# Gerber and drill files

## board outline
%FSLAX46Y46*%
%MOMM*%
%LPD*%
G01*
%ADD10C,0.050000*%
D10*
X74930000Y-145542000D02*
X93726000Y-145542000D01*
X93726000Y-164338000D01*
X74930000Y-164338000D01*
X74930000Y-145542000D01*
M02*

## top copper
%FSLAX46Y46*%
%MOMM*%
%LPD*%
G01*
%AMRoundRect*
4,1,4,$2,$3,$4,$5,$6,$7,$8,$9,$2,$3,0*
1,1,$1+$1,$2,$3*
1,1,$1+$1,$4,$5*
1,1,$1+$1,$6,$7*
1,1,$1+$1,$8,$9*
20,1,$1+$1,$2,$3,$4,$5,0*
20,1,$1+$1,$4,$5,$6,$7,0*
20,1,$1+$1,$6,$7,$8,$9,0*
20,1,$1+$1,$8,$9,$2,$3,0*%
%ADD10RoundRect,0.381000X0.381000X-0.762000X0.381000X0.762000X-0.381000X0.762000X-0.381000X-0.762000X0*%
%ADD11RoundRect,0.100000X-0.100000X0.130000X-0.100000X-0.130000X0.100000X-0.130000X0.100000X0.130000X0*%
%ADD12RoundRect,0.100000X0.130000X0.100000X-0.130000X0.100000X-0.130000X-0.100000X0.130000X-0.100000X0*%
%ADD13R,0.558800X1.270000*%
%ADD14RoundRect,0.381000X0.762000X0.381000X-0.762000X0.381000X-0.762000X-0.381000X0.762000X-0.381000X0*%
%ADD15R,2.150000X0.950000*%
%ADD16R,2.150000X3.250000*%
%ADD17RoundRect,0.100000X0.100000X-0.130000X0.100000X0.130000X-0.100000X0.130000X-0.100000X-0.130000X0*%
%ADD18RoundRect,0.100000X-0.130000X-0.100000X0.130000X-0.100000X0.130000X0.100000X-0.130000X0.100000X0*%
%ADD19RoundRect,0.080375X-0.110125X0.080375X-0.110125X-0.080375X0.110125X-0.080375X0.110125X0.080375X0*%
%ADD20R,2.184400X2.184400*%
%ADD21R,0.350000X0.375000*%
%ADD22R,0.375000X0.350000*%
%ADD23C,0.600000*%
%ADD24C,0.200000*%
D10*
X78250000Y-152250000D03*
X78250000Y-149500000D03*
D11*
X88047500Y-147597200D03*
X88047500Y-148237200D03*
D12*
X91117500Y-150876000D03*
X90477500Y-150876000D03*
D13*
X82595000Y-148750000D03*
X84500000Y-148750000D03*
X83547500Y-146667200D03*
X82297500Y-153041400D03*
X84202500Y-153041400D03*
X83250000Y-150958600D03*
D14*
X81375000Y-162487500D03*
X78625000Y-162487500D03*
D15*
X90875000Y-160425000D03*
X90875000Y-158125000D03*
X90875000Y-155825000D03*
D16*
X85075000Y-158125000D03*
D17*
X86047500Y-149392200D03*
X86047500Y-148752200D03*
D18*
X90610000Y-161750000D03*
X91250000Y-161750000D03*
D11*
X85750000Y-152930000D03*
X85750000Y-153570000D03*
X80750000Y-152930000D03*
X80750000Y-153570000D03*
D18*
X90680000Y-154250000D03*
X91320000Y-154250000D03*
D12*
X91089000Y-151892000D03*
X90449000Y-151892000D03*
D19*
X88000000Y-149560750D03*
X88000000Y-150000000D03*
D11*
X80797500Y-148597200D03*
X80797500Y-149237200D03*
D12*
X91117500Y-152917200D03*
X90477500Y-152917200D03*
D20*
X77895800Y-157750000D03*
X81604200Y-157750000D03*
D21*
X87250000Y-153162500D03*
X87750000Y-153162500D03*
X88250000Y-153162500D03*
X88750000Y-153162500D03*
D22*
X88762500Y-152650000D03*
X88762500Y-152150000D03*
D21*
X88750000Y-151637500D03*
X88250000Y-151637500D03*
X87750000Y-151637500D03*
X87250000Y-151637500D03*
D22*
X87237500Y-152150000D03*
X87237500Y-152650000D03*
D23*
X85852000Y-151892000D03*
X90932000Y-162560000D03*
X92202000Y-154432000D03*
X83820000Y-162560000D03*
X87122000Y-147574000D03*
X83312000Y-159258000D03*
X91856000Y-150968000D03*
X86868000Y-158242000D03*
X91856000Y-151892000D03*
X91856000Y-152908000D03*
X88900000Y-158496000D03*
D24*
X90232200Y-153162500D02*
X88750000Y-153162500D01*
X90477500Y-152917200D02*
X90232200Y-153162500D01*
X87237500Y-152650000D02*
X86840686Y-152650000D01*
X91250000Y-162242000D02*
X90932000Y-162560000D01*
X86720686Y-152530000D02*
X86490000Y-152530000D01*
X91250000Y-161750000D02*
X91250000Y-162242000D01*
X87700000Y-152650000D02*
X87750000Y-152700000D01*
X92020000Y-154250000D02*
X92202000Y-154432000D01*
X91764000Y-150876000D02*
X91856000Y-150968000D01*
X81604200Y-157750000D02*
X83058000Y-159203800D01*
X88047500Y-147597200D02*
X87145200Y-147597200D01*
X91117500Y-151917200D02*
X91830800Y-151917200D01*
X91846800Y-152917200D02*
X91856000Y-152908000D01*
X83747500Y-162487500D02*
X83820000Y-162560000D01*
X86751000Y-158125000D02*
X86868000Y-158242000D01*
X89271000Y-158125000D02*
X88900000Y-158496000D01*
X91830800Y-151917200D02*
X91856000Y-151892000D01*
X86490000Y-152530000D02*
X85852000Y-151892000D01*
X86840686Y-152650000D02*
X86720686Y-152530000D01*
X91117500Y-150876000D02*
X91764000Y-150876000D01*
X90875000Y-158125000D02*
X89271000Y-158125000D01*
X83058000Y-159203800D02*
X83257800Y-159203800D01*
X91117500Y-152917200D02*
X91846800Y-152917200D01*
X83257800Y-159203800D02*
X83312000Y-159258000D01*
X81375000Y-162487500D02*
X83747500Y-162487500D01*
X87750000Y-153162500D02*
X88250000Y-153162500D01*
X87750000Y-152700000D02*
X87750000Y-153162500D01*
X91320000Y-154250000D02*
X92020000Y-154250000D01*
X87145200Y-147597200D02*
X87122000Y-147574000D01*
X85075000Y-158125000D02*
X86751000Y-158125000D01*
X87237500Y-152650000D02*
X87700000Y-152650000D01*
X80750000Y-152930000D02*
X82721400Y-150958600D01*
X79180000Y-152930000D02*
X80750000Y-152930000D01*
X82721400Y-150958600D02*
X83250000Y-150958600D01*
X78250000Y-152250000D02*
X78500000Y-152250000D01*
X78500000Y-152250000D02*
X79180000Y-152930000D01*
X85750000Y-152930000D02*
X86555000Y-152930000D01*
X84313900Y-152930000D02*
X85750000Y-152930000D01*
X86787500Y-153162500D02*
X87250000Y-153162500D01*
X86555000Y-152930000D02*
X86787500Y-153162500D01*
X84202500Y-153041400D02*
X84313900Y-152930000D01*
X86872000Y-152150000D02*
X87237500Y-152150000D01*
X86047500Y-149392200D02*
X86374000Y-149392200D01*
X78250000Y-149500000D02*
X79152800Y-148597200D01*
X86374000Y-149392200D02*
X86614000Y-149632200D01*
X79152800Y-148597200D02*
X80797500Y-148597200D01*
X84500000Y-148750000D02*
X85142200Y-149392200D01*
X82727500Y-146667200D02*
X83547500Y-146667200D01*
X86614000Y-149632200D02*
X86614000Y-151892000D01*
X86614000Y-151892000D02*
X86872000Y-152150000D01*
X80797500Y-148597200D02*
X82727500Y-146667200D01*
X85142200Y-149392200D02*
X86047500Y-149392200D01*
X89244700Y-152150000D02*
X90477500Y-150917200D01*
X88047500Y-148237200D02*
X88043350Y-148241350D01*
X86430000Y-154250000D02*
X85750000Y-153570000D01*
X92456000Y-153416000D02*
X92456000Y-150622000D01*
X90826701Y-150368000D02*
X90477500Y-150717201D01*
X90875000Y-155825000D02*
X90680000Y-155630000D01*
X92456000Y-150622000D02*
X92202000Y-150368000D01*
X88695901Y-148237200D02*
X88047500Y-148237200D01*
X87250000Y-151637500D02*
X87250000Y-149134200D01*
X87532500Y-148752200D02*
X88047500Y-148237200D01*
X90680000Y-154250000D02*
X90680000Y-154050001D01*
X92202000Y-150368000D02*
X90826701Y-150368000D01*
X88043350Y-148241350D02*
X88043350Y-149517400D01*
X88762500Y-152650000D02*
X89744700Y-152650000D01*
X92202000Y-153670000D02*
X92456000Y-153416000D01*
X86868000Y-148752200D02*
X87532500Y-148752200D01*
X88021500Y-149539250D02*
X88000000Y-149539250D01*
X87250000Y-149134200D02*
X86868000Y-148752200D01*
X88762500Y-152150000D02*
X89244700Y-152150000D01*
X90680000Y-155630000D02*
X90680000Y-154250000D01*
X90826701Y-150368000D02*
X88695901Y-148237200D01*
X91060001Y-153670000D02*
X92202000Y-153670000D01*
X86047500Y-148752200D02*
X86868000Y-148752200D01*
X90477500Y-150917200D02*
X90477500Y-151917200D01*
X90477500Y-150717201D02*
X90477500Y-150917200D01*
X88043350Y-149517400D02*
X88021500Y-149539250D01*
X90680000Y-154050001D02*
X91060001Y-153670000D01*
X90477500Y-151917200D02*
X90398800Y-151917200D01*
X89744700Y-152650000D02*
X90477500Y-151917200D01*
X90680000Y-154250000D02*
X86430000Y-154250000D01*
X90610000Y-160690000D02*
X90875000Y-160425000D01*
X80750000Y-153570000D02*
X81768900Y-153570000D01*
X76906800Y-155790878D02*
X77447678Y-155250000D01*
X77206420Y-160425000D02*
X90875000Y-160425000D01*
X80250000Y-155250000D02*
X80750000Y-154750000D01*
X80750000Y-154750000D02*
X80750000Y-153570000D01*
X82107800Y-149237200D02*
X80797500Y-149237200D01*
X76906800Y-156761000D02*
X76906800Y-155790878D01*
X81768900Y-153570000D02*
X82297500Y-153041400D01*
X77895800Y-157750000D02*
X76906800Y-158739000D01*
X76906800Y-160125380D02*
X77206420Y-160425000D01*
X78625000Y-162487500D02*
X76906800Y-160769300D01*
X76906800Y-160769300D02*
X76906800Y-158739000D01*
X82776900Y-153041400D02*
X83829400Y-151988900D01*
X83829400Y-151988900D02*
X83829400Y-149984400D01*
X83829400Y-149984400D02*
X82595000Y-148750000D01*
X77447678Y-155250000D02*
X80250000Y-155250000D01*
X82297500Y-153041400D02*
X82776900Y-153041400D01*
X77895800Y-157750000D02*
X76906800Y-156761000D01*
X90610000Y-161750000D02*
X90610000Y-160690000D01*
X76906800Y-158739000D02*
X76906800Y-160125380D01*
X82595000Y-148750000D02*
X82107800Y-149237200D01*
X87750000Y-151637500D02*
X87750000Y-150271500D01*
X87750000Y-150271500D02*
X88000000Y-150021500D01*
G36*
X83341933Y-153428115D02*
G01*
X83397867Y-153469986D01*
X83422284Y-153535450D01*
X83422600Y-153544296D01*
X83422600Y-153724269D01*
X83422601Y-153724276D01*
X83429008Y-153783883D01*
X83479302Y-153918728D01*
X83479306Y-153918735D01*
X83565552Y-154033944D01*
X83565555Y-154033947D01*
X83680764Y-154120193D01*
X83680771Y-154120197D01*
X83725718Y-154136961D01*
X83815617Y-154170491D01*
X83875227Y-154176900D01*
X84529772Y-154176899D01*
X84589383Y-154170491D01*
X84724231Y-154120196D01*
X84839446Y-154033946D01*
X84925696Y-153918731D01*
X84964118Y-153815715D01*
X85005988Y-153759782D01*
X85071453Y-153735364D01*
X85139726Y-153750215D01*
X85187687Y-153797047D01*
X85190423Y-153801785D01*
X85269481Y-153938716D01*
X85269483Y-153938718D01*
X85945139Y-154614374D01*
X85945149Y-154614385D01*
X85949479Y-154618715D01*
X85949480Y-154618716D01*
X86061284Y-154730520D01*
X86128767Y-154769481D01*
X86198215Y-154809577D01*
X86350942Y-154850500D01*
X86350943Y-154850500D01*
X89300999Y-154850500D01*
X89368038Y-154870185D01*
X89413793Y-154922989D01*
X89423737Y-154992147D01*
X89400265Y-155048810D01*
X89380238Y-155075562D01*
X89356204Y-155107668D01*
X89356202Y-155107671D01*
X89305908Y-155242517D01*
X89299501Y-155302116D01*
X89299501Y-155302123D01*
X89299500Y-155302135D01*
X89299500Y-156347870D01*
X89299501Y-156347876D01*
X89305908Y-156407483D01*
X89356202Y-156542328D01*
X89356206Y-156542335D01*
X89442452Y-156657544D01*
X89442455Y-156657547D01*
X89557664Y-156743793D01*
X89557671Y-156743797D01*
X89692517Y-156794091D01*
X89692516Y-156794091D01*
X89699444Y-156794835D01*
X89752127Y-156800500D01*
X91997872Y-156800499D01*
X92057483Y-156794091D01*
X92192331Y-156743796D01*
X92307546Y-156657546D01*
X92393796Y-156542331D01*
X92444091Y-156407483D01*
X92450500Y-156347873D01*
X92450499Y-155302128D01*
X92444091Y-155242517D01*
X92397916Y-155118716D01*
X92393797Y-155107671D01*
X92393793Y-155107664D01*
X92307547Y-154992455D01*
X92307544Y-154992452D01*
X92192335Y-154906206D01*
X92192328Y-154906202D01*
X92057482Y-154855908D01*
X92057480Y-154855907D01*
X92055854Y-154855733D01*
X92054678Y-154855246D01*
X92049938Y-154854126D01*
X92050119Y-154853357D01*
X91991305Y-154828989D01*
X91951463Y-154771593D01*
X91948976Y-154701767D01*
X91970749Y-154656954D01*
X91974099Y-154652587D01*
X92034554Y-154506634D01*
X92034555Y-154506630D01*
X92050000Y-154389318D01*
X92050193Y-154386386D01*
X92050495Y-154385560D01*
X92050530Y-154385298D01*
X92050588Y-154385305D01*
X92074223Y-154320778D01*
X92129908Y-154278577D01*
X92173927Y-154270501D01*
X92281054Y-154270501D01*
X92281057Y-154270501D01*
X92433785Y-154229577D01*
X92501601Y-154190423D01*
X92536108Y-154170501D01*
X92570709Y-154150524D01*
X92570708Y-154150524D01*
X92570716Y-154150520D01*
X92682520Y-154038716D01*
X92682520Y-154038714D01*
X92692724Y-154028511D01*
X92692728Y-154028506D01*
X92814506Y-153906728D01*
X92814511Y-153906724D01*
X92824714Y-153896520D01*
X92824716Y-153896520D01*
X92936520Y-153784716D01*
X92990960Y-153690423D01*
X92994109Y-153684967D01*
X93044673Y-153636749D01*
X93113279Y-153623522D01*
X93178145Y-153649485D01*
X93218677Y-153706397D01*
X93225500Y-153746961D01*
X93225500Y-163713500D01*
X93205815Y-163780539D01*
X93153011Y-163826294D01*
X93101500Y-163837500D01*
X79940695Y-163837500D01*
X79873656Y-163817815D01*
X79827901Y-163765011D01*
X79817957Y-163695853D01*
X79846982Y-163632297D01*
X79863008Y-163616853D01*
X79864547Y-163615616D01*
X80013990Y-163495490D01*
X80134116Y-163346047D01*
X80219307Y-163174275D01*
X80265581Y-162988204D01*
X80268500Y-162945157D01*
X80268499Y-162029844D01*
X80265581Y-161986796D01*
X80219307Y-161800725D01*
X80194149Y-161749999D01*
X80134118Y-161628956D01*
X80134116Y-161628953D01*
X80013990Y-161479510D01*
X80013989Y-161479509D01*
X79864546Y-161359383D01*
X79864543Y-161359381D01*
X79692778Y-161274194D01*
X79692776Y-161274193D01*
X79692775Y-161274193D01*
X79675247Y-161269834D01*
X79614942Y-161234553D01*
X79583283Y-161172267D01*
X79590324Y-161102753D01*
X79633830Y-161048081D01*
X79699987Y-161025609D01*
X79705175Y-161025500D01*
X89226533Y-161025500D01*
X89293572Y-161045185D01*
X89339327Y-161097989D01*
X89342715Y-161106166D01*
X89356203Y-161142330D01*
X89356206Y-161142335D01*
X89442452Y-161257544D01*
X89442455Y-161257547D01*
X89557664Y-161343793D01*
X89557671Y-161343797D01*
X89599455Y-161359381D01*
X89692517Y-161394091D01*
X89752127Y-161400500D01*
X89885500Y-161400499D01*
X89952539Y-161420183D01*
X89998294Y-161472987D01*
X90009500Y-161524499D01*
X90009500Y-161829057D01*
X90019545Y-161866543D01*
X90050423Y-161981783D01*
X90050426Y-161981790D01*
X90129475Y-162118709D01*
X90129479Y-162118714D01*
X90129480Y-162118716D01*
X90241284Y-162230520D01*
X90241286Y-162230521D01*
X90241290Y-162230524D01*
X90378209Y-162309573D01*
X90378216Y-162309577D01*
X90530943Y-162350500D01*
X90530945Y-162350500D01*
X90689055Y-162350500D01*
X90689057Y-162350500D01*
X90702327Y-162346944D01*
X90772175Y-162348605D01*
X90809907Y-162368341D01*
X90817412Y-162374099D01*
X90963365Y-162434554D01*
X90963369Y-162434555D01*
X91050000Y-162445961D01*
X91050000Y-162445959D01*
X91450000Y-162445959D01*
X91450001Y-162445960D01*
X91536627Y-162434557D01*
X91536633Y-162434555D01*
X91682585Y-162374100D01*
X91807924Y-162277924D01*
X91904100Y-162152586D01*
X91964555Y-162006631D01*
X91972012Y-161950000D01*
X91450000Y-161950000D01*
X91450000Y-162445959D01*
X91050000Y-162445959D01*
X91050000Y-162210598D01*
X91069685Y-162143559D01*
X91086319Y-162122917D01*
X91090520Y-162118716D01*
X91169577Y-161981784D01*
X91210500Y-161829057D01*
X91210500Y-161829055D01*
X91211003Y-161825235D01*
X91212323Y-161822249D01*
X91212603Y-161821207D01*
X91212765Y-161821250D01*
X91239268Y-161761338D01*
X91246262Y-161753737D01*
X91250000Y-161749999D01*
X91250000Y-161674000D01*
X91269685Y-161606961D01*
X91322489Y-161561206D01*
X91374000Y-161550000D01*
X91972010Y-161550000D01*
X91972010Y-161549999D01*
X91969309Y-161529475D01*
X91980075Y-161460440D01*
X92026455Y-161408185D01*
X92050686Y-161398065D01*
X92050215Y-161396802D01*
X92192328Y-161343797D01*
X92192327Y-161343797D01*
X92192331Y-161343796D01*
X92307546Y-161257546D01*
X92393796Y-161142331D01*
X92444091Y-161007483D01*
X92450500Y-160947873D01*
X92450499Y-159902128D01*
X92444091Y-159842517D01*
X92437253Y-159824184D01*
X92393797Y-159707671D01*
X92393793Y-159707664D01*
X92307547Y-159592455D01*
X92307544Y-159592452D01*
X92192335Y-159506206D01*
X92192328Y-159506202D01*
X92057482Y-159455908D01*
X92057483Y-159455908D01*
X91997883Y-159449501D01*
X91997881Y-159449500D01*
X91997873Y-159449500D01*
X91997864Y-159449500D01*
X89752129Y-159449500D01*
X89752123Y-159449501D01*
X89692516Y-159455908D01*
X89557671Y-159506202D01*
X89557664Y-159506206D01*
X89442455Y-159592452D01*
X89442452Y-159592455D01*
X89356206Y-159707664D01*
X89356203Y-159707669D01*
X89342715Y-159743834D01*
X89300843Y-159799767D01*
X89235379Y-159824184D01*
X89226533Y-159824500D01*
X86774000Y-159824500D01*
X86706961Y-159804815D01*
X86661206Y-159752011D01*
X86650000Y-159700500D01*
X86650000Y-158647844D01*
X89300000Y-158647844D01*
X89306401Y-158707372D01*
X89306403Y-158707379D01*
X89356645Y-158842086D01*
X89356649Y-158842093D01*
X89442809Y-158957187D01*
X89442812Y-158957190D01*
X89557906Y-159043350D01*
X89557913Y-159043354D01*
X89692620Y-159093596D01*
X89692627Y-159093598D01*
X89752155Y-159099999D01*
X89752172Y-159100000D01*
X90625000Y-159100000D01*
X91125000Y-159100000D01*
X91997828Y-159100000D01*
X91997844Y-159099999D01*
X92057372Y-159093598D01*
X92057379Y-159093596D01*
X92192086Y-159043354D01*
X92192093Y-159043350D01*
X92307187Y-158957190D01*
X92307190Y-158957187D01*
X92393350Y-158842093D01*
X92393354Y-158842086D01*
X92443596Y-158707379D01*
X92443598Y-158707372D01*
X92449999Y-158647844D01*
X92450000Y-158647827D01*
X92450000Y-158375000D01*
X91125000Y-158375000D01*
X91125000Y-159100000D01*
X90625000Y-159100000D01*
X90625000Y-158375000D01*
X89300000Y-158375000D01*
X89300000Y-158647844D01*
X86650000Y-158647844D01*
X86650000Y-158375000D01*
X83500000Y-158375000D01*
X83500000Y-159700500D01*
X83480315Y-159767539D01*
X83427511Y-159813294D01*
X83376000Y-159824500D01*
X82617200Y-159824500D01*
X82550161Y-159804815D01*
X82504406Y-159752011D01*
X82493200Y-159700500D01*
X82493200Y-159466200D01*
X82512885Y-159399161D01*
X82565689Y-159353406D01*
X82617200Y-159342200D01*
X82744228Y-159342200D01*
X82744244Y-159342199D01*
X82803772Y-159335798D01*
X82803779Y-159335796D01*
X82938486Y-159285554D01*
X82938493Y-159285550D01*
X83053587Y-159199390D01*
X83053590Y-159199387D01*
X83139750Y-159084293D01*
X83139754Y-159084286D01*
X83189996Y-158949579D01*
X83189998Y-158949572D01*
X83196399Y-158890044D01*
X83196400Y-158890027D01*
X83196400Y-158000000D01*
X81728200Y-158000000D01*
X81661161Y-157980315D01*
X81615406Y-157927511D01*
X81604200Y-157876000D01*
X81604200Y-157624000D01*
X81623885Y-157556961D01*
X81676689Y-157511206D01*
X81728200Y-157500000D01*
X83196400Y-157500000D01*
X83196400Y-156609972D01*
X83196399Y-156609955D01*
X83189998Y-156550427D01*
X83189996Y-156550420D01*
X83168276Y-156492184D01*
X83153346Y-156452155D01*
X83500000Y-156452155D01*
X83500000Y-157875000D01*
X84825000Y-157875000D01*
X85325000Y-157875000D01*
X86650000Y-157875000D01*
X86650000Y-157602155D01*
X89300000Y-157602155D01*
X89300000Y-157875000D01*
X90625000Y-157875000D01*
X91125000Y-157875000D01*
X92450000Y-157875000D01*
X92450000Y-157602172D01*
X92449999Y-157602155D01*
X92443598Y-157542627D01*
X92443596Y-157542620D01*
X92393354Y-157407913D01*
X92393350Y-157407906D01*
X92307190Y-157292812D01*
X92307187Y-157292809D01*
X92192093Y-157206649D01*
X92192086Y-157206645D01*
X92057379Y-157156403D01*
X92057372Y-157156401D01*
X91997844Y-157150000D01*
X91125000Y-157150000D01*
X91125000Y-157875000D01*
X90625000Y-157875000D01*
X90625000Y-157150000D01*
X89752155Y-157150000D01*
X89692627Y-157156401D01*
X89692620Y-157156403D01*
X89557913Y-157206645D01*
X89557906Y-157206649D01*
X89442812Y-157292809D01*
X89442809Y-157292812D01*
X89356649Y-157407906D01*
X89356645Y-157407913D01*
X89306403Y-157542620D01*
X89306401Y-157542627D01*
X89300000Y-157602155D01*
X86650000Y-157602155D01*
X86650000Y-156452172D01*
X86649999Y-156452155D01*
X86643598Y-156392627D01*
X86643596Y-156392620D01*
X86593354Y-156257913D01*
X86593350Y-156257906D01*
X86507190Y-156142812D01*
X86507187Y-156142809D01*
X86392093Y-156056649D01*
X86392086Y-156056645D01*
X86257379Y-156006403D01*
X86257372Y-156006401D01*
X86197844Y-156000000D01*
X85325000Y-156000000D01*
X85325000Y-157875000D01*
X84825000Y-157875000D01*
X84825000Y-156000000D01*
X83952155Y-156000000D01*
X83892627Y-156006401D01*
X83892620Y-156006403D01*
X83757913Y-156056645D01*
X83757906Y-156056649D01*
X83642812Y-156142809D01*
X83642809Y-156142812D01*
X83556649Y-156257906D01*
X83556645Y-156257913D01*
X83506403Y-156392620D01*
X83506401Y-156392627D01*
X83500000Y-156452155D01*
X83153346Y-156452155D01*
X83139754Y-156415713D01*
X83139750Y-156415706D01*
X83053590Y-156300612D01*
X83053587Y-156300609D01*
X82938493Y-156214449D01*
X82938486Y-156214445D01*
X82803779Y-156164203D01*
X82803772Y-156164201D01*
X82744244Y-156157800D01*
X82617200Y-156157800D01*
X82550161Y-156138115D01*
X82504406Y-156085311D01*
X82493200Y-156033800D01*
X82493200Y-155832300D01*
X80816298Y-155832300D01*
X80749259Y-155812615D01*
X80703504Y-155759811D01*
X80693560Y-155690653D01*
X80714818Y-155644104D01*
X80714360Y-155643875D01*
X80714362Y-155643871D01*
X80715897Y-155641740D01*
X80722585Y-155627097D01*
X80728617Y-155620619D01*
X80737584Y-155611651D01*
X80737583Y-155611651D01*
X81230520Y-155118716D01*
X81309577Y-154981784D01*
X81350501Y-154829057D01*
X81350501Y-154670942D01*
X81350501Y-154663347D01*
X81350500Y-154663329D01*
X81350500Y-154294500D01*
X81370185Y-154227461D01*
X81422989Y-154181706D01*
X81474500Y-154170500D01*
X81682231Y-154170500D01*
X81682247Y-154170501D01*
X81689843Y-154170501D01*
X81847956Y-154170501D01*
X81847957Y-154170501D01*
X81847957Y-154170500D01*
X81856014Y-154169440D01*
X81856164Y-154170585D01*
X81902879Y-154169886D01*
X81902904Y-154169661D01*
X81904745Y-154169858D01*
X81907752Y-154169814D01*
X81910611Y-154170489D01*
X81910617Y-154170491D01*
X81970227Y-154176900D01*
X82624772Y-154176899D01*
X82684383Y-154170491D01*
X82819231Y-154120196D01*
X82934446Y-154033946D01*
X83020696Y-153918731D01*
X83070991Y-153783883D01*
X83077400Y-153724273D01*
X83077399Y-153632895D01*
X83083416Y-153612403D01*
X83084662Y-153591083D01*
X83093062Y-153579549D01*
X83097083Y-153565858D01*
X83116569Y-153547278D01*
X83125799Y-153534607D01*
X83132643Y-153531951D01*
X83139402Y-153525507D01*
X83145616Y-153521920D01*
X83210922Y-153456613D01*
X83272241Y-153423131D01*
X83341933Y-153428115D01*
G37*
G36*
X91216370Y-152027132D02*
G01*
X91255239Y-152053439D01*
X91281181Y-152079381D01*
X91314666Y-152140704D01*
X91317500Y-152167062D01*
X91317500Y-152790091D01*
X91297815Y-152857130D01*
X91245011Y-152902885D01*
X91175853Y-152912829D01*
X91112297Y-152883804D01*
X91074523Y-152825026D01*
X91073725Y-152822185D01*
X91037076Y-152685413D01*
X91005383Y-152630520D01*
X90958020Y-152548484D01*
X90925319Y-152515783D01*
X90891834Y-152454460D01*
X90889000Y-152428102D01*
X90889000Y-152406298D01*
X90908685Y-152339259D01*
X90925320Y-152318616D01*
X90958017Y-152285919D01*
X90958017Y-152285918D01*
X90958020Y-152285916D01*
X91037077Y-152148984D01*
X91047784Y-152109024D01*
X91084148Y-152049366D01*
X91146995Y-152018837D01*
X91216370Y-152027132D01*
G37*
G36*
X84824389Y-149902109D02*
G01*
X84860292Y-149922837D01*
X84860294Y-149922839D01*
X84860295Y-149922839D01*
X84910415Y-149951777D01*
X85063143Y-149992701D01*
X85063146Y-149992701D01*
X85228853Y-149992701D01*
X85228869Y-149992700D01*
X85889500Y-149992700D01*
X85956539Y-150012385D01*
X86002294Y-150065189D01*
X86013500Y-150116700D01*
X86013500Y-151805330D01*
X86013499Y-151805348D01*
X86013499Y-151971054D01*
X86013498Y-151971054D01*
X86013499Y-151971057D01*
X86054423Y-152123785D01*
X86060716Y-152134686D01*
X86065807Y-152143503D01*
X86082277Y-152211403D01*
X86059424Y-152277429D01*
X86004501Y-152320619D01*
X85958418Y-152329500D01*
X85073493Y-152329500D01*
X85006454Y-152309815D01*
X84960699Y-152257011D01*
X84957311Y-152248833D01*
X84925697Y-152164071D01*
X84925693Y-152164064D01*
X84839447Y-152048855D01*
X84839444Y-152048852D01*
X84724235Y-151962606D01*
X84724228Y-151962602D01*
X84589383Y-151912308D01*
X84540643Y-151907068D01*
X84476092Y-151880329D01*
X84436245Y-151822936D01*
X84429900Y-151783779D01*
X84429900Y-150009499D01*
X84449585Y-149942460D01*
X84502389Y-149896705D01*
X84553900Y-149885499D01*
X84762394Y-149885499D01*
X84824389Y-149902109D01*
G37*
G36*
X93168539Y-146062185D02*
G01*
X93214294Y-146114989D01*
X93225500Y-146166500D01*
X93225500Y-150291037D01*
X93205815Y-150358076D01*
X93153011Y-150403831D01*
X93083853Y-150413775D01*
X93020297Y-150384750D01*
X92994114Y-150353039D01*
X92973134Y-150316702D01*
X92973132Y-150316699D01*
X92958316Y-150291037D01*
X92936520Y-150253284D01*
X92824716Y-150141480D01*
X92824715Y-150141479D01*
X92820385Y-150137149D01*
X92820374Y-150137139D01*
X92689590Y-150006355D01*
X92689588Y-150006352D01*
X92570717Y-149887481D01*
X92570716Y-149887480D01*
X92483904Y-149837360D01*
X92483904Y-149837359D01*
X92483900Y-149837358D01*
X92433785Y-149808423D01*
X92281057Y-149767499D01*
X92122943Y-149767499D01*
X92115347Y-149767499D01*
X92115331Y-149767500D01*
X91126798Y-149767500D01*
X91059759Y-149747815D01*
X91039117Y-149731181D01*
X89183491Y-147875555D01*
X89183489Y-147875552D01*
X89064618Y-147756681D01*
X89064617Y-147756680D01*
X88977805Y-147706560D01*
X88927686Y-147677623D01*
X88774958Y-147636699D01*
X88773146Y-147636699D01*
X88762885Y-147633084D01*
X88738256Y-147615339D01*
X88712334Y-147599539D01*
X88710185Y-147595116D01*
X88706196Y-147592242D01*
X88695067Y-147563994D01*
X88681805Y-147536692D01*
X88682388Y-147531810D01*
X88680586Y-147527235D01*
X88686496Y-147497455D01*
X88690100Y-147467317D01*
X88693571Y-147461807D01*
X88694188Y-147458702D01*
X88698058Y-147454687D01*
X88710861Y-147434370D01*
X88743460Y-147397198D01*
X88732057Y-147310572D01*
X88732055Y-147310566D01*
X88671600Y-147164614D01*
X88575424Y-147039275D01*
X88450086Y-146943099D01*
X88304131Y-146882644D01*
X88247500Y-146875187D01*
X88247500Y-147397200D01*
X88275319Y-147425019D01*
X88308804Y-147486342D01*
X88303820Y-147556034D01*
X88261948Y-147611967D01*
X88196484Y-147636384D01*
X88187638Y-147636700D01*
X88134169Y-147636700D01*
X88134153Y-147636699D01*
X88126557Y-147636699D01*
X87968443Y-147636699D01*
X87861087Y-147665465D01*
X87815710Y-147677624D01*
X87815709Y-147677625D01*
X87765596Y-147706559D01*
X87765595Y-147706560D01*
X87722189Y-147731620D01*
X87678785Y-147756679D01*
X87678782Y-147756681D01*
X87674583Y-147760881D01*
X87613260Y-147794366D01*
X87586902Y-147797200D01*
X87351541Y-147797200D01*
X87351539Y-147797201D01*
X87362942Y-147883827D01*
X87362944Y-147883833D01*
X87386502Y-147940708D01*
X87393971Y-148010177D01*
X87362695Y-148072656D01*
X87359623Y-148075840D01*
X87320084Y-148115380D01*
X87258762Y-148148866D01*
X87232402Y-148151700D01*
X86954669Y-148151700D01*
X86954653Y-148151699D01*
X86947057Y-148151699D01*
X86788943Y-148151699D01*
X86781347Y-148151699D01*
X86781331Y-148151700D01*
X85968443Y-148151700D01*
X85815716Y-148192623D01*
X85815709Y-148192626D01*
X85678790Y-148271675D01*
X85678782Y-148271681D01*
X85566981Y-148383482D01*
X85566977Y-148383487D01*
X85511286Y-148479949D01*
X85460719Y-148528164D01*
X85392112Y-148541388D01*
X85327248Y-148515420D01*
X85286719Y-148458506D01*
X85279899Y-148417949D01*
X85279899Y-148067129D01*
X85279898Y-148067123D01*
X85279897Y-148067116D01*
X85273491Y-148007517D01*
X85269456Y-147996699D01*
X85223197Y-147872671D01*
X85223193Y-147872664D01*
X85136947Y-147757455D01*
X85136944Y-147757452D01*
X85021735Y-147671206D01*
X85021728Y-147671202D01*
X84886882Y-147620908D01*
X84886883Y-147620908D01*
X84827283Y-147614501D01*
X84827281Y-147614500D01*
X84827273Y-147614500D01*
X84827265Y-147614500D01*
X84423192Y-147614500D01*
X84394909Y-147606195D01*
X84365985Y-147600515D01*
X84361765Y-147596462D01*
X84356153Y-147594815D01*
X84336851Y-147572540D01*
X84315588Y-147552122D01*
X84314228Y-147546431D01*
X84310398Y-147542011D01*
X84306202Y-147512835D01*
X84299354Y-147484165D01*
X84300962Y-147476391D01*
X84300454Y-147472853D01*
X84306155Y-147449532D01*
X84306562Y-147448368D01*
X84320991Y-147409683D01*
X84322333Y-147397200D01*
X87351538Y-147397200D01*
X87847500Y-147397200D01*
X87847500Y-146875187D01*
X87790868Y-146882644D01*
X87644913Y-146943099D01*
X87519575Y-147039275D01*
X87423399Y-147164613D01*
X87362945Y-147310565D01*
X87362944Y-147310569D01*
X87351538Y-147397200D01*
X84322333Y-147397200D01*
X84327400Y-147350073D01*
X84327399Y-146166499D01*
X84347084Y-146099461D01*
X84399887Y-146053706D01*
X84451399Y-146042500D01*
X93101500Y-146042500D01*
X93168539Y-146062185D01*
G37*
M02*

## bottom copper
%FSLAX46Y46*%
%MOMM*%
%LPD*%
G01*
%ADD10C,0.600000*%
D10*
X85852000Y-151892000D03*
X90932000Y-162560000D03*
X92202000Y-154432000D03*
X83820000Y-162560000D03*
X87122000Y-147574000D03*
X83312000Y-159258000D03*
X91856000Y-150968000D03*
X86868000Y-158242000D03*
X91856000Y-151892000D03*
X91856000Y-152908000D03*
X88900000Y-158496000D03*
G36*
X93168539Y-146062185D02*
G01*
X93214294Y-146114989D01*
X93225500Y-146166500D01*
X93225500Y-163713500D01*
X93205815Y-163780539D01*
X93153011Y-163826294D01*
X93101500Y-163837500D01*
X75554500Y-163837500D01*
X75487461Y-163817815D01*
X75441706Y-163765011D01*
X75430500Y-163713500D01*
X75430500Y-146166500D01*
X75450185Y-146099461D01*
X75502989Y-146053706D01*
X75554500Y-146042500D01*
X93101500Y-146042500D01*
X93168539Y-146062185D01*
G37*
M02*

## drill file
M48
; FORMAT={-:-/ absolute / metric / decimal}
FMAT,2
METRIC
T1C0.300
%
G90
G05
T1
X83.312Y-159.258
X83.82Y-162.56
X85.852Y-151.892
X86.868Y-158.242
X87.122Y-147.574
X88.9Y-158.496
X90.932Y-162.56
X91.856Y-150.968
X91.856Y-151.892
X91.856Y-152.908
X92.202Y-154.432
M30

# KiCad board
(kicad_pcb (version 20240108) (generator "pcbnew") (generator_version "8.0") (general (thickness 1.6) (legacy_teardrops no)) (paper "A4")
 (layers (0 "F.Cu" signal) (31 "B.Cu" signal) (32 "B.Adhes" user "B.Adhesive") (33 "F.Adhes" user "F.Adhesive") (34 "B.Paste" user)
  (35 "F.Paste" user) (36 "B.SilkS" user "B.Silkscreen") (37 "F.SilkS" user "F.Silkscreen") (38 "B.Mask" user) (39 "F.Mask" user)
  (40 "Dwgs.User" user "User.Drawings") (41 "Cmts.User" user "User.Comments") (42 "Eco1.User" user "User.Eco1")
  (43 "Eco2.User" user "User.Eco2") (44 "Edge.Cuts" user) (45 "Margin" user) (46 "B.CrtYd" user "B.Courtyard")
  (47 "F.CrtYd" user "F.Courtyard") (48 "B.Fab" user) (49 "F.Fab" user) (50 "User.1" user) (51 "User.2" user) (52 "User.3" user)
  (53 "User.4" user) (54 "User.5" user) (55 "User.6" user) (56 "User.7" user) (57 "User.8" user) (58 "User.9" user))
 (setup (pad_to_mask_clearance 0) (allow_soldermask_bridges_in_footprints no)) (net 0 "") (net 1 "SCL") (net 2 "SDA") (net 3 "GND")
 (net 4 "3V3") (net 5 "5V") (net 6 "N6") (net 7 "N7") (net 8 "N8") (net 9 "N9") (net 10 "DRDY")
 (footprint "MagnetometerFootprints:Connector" (layer "F.Cu") (at 81.5 149.25 90)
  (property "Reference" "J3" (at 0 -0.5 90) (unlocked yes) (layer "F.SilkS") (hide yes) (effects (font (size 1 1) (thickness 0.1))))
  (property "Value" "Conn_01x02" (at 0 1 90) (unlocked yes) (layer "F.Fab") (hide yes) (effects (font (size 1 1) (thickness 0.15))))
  (pad "1" smd roundrect (at -3 -3.25 90) (size 2.286 1.524) (layers "F.Cu" "F.Mask") (roundrect_rratio 0.25) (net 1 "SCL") (zone_connect 2)
   (thermal_bridge_angle 45))
  (pad "2" smd roundrect (at -0.25 -3.25 90) (size 2.286 1.524) (layers "F.Cu" "F.Mask") (roundrect_rratio 0.25) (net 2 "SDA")
   (zone_connect 2) (thermal_bridge_angle 45)))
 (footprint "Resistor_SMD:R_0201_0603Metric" (layer "F.Cu") (at 88.0475 147.9172 -90)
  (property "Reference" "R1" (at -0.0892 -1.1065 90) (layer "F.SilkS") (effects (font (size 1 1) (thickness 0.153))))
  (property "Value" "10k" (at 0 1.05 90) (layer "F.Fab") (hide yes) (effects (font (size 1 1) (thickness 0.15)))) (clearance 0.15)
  (pad "" smd roundrect (at -0.345 0 270) (size 0.318 0.36) (layers "F.Paste") (roundrect_rratio 0.25))
  (pad "" smd roundrect (at 0.345 0 270) (size 0.318 0.36) (layers "F.Paste") (roundrect_rratio 0.25))
  (pad "1" smd roundrect (at -0.32 0 270) (size 0.46 0.4) (layers "F.Cu" "F.Mask") (roundrect_rratio 0.25) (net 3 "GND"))
  (pad "2" smd roundrect (at 0.32 0 270) (size 0.46 0.4) (layers "F.Cu" "F.Mask") (roundrect_rratio 0.25) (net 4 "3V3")))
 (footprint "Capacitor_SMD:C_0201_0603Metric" (layer "F.Cu") (at 90.7975 150.876 180)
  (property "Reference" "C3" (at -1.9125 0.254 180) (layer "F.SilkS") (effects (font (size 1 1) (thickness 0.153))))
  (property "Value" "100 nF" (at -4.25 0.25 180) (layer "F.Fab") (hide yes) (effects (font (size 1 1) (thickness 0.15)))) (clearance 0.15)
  (pad "" smd roundrect (at -0.345 0 180) (size 0.318 0.36) (layers "F.Paste") (roundrect_rratio 0.25))
  (pad "" smd roundrect (at 0.345 0 180) (size 0.318 0.36) (layers "F.Paste") (roundrect_rratio 0.25))
  (pad "1" smd roundrect (at -0.32 0 180) (size 0.46 0.4) (layers "F.Cu" "F.Mask") (roundrect_rratio 0.25) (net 3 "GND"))
  (pad "2" smd roundrect (at 0.32 0 180) (size 0.46 0.4) (layers "F.Cu" "F.Mask") (roundrect_rratio 0.25) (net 4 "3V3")))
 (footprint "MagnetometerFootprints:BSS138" (layer "F.Cu") (at 83.5475 147.7086)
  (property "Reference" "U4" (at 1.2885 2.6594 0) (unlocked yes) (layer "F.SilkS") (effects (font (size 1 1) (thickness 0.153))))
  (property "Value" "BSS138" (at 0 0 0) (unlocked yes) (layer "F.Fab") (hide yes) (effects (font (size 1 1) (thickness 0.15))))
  (pad "1" smd rect (at -0.9525 1.0414) (size 0.5588 1.27) (layers "F.Cu" "F.Paste" "F.Mask") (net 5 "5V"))
  (pad "2" smd rect (at 0.9525 1.0414) (size 0.5588 1.27) (layers "F.Cu" "F.Paste" "F.Mask") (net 2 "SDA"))
  (pad "3" smd rect (at 0 -1.0414) (size 0.5588 1.27) (layers "F.Cu" "F.Paste" "F.Mask") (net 2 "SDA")))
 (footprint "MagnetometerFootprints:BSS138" (layer "F.Cu") (at 83.25 152)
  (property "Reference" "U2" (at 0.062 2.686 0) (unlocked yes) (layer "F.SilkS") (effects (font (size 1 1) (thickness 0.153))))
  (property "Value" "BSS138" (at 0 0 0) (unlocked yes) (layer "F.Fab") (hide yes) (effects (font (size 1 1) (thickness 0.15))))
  (pad "1" smd rect (at -0.9525 1.0414) (size 0.5588 1.27) (layers "F.Cu" "F.Paste" "F.Mask") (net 5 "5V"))
  (pad "2" smd rect (at 0.9525 1.0414) (size 0.5588 1.27) (layers "F.Cu" "F.Paste" "F.Mask") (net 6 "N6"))
  (pad "3" smd rect (at 0 -1.0414) (size 0.5588 1.27) (layers "F.Cu" "F.Paste" "F.Mask") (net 1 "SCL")))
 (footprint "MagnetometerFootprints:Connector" (layer "F.Cu") (at 78.375 159.2375 180)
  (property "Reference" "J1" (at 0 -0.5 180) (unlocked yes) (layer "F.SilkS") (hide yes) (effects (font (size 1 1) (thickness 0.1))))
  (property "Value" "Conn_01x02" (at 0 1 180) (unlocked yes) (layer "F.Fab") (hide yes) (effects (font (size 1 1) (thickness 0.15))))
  (pad "1" smd roundrect (at -3 -3.25 180) (size 2.286 1.524) (layers "F.Cu" "F.Mask") (roundrect_rratio 0.25) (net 3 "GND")
   (zone_connect 2) (thermal_bridge_angle 45))
  (pad "2" smd roundrect (at -0.25 -3.25 180) (size 2.286 1.524) (layers "F.Cu" "F.Mask") (roundrect_rratio 0.25) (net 5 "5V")
   (zone_connect 2) (thermal_bridge_angle 45)))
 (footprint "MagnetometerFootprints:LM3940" (layer "F.Cu") (at 87.5 155 180)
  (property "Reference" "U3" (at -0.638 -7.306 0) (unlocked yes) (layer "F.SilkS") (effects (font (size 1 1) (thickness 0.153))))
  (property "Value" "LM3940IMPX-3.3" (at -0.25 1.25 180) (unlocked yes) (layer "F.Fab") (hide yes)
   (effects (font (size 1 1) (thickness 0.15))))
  (pad "1" smd rect (at -3.375 -5.425 180) (size 2.15 0.95) (layers "F.Cu" "F.Paste" "F.Mask") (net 5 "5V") (solder_mask_margin 0.102))
  (pad "2" smd rect (at -3.375 -3.125 180) (size 2.15 0.95) (layers "F.Cu" "F.Paste" "F.Mask") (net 3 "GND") (solder_mask_margin 0.102))
  (pad "3" smd rect (at -3.375 -0.825 180) (size 2.15 0.95) (layers "F.Cu" "F.Paste" "F.Mask") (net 4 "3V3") (solder_mask_margin 0.102))
  (pad "4" smd rect (at 2.425 -3.125 180) (size 2.15 3.25) (layers "F.Cu" "F.Paste" "F.Mask") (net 3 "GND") (solder_mask_margin 0.102)))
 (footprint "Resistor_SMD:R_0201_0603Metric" (layer "F.Cu") (at 86.0475 149.0722 90)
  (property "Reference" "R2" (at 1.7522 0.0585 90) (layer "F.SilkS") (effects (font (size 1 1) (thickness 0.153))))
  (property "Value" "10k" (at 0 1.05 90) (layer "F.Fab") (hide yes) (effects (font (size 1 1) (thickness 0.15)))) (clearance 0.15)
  (pad "" smd roundrect (at -0.345 0 90) (size 0.318 0.36) (layers "F.Paste") (roundrect_rratio 0.25))
  (pad "" smd roundrect (at 0.345 0 90) (size 0.318 0.36) (layers "F.Paste") (roundrect_rratio 0.25))
  (pad "1" smd roundrect (at -0.32 0 90) (size 0.46 0.4) (layers "F.Cu" "F.Mask") (roundrect_rratio 0.25) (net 2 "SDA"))
  (pad "2" smd roundrect (at 0.32 0 90) (size 0.46 0.4) (layers "F.Cu" "F.Mask") (roundrect_rratio 0.25) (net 4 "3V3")))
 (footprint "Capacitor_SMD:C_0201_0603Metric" (layer "F.Cu") (at 90.93 161.75)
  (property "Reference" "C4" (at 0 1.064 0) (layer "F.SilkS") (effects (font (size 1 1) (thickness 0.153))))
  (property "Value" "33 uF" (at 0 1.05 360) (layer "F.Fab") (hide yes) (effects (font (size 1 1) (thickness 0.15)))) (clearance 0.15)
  (pad "" smd roundrect (at -0.345 0) (size 0.318 0.36) (layers "F.Paste") (roundrect_rratio 0.25))
  (pad "" smd roundrect (at 0.345 0) (size 0.318 0.36) (layers "F.Paste") (roundrect_rratio 0.25))
  (pad "1" smd roundrect (at -0.32 0) (size 0.46 0.4) (layers "F.Cu" "F.Mask") (roundrect_rratio 0.25) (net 5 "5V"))
  (pad "2" smd roundrect (at 0.32 0) (size 0.46 0.4) (layers "F.Cu" "F.Mask") (roundrect_rratio 0.25) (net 3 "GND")))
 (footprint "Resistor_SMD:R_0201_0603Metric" (layer "F.Cu") (at 85.75 153.25 -90)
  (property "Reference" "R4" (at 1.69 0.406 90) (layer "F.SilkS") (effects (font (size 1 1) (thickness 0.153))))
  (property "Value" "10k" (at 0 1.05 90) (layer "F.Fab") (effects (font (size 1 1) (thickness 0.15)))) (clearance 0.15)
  (pad "" smd roundrect (at -0.345 0 270) (size 0.318 0.36) (layers "F.Paste") (roundrect_rratio 0.25))
  (pad "" smd roundrect (at 0.345 0 270) (size 0.318 0.36) (layers "F.Paste") (roundrect_rratio 0.25))
  (pad "1" smd roundrect (at -0.32 0 270) (size 0.46 0.4) (layers "F.Cu" "F.Mask") (roundrect_rratio 0.25) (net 6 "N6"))
  (pad "2" smd roundrect (at 0.32 0 270) (size 0.46 0.4) (layers "F.Cu" "F.Mask") (roundrect_rratio 0.25) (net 4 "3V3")))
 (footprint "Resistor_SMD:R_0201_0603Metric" (layer "F.Cu") (at 80.75 153.25 -90)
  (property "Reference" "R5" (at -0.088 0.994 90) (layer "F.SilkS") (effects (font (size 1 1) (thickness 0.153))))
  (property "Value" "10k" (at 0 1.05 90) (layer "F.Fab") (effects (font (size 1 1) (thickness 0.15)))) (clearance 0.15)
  (pad "" smd roundrect (at -0.345 0 270) (size 0.318 0.36) (layers "F.Paste") (roundrect_rratio 0.25))
  (pad "" smd roundrect (at 0.345 0 270) (size 0.318 0.36) (layers "F.Paste") (roundrect_rratio 0.25))
  (pad "1" smd roundrect (at -0.32 0 270) (size 0.46 0.4) (layers "F.Cu" "F.Mask") (roundrect_rratio 0.25) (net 1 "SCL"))
  (pad "2" smd roundrect (at 0.32 0 270) (size 0.46 0.4) (layers "F.Cu" "F.Mask") (roundrect_rratio 0.25) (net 5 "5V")))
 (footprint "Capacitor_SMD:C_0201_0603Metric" (layer "F.Cu") (at 91 154.25)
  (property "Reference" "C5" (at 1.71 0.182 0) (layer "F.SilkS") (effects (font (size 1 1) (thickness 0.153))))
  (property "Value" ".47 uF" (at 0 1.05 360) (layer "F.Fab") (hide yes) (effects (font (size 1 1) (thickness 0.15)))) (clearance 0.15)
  (pad "" smd roundrect (at -0.345 0) (size 0.318 0.36) (layers "F.Paste") (roundrect_rratio 0.25))
  (pad "" smd roundrect (at 0.345 0) (size 0.318 0.36) (layers "F.Paste") (roundrect_rratio 0.25))
  (pad "1" smd roundrect (at -0.32 0) (size 0.46 0.4) (layers "F.Cu" "F.Mask") (roundrect_rratio 0.25) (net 4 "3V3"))
  (pad "2" smd roundrect (at 0.32 0) (size 0.46 0.4) (layers "F.Cu" "F.Mask") (roundrect_rratio 0.25) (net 3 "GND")))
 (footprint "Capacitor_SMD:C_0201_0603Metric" (layer "F.Cu") (at 90.769 151.892 180)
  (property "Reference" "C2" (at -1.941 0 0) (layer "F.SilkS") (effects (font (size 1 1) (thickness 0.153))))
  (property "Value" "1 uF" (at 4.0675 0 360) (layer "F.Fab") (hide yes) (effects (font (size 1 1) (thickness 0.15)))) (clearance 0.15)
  (pad "" smd roundrect (at -0.345 0 180) (size 0.318 0.36) (layers "F.Paste") (roundrect_rratio 0.25))
  (pad "" smd roundrect (at 0.345 0 180) (size 0.318 0.36) (layers "F.Paste") (roundrect_rratio 0.25))
  (pad "1" smd roundrect (at -0.32 0 180) (size 0.46 0.4) (layers "F.Cu" "F.Mask") (roundrect_rratio 0.25) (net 3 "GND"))
  (pad "2" smd roundrect (at 0.32 0 180) (size 0.46 0.4) (layers "F.Cu" "F.Mask") (roundrect_rratio 0.25) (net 4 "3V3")))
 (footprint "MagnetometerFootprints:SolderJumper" (layer "F.Cu") (at 85.8095 153.9 -90)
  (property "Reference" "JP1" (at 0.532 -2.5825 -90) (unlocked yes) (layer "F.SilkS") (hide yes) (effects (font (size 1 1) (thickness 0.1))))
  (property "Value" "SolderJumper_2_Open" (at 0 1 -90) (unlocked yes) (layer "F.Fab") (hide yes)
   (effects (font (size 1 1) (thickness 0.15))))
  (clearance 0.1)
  (pad "1" smd roundrect (at -4.33925 -2.1905 270) (size 0.3215 0.381) (layers "F.Cu" "F.Paste" "F.Mask") (roundrect_rratio 0.25)
   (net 4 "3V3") (thermal_bridge_angle 45))
  (pad "2" smd roundrect (at -3.9 -2.1905 270) (size 0.3215 0.381) (layers "F.Cu" "F.Paste" "F.Mask") (roundrect_rratio 0.25) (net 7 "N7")
   (thermal_bridge_angle 45)))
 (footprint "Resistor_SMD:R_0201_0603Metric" (layer "F.Cu") (at 80.7975 148.9172 -90)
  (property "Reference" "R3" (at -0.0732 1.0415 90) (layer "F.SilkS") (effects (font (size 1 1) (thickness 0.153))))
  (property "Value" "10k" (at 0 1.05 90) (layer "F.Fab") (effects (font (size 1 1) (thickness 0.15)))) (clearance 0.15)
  (pad "" smd roundrect (at -0.345 0 270) (size 0.318 0.36) (layers "F.Paste") (roundrect_rratio 0.25))
  (pad "" smd roundrect (at 0.345 0 270) (size 0.318 0.36) (layers "F.Paste") (roundrect_rratio 0.25))
  (pad "1" smd roundrect (at -0.32 0 270) (size 0.46 0.4) (layers "F.Cu" "F.Mask") (roundrect_rratio 0.25) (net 2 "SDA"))
  (pad "2" smd roundrect (at 0.32 0 270) (size 0.46 0.4) (layers "F.Cu" "F.Mask") (roundrect_rratio 0.25) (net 5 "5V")))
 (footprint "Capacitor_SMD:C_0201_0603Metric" (layer "F.Cu") (at 90.7975 152.9172 180)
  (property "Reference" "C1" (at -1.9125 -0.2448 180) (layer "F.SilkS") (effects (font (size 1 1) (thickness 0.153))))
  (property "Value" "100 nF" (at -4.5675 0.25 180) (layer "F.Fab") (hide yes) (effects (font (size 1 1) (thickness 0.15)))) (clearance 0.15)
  (pad "" smd roundrect (at -0.345 0 180) (size 0.318 0.36) (layers "F.Paste") (roundrect_rratio 0.25))
  (pad "" smd roundrect (at 0.345 0 180) (size 0.318 0.36) (layers "F.Paste") (roundrect_rratio 0.25))
  (pad "1" smd roundrect (at -0.32 0 180) (size 0.46 0.4) (layers "F.Cu" "F.Mask") (roundrect_rratio 0.25) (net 3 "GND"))
  (pad "2" smd roundrect (at 0.32 0 180) (size 0.46 0.4) (layers "F.Cu" "F.Mask") (roundrect_rratio 0.25) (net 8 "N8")))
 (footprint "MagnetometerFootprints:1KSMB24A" (layer "F.Cu") (at 79.75 157.75)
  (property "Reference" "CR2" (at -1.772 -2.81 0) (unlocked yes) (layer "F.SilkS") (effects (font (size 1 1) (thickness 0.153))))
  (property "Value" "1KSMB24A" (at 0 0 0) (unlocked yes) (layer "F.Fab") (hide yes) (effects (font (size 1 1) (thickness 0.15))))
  (pad "1" smd rect (at -1.8542 0 90) (size 2.1844 2.1844) (layers "F.Cu" "F.Paste" "F.Mask") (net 5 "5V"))
  (pad "2" smd rect (at 1.8542 0 90) (size 2.1844 2.1844) (layers "F.Cu" "F.Paste" "F.Mask") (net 3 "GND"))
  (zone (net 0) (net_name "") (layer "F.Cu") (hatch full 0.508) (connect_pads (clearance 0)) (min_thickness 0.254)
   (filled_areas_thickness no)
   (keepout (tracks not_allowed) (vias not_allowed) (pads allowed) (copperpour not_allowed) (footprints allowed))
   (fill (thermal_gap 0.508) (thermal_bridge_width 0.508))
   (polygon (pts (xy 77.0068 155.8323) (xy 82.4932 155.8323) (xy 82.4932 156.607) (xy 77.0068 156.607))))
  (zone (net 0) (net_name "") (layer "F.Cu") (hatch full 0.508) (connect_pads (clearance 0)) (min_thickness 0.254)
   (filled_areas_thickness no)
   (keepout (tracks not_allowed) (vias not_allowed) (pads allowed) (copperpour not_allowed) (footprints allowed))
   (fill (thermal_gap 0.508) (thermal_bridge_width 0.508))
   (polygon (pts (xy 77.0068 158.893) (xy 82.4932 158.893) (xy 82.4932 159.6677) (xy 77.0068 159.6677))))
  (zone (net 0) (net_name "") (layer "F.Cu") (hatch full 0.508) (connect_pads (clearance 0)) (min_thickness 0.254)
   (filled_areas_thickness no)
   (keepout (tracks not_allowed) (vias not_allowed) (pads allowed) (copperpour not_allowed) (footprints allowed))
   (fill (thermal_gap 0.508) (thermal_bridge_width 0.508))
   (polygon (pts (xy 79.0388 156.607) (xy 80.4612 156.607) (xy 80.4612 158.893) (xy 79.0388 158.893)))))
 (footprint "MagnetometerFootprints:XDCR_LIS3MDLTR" (layer "F.Cu") (at 88 152.4 90)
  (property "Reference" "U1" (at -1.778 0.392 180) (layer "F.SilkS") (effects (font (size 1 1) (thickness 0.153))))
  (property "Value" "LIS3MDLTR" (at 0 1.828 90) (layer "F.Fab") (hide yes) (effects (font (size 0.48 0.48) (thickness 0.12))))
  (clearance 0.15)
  (pad "1" smd rect (at -0.7625 -0.75 90) (size 0.375 0.35) (layers "F.Cu" "F.Paste") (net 6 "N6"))
  (pad "2" smd rect (at -0.7625 -0.25 90) (size 0.375 0.35) (layers "F.Cu" "F.Paste") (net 3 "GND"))
  (pad "3" smd rect (at -0.7625 0.25 90) (size 0.375 0.35) (layers "F.Cu" "F.Paste") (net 3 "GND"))
  (pad "4" smd rect (at -0.7625 0.75 90) (size 0.375 0.35) (layers "F.Cu" "F.Paste") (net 8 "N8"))
  (pad "5" smd rect (at -0.25 0.7625 90) (size 0.35 0.375) (layers "F.Cu" "F.Paste") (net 4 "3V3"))
  (pad "6" smd rect (at 0.25 0.7625 90) (size 0.35 0.375) (layers "F.Cu" "F.Paste") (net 4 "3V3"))
  (pad "7" smd rect (at 0.7625 0.75 90) (size 0.375 0.35) (layers "F.Cu" "F.Paste") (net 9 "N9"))
  (pad "8" smd rect (at 0.7625 0.25 90) (size 0.375 0.35) (layers "F.Cu" "F.Paste") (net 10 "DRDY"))
  (pad "9" smd rect (at 0.7625 -0.25 90) (size 0.375 0.35) (layers "F.Cu" "F.Paste") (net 7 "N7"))
  (pad "10" smd rect (at 0.7625 -0.75 90) (size 0.375 0.35) (layers "F.Cu" "F.Paste") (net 4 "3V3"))
  (pad "11" smd rect (at 0.25 -0.7625 90) (size 0.35 0.375) (layers "F.Cu" "F.Paste") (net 2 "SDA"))
  (pad "12" smd rect (at -0.25 -0.7625 90) (size 0.35 0.375) (layers "F.Cu" "F.Paste") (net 3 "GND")))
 (gr_rect (start 74.93 145.542) (end 93.726 164.338) (stroke (width 0.05) (type default)) (fill none) (layer "Edge.Cuts"))
 (segment (start 90.2322 153.1625) (end 88.75 153.1625) (width 0.2) (layer "F.Cu") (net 8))
 (segment (start 90.4775 152.9172) (end 90.2322 153.1625) (width 0.2) (layer "F.Cu") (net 8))
 (segment (start 87.2375 152.65) (end 86.840686 152.65) (width 0.2) (layer "F.Cu") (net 3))
 (segment (start 91.25 162.242) (end 90.932 162.56) (width 0.2) (layer "F.Cu") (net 3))
 (segment (start 86.720686 152.53) (end 86.49 152.53) (width 0.2) (layer "F.Cu") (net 3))
 (segment (start 91.25 161.75) (end 91.25 162.242) (width 0.2) (layer "F.Cu") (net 3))
 (segment (start 87.7 152.65) (end 87.75 152.7) (width 0.2) (layer "F.Cu") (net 3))
 (segment (start 92.02 154.25) (end 92.202 154.432) (width 0.2) (layer "F.Cu") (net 3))
 (segment (start 91.764 150.876) (end 91.856 150.968) (width 0.2) (layer "F.Cu") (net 3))
 (segment (start 81.6042 157.75) (end 83.058 159.2038) (width 0.2) (layer "F.Cu") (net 3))
 (segment (start 88.0475 147.5972) (end 87.1452 147.5972) (width 0.2) (layer "F.Cu") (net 3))
 (segment (start 91.1175 151.9172) (end 91.8308 151.9172) (width 0.2) (layer "F.Cu") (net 3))
 (segment (start 91.8468 152.9172) (end 91.856 152.908) (width 0.2) (layer "F.Cu") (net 3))
 (segment (start 83.7475 162.4875) (end 83.82 162.56) (width 0.2) (layer "F.Cu") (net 3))
 (segment (start 86.751 158.125) (end 86.868 158.242) (width 0.2) (layer "F.Cu") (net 3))
 (segment (start 89.271 158.125) (end 88.9 158.496) (width 0.2) (layer "F.Cu") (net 3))
 (segment (start 91.8308 151.9172) (end 91.856 151.892) (width 0.2) (layer "F.Cu") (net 3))
 (segment (start 86.49 152.53) (end 85.852 151.892) (width 0.2) (layer "F.Cu") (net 3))
 (segment (start 86.840686 152.65) (end 86.720686 152.53) (width 0.2) (layer "F.Cu") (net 3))
 (segment (start 91.1175 150.876) (end 91.764 150.876) (width 0.2) (layer "F.Cu") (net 3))
 (segment (start 90.875 158.125) (end 89.271 158.125) (width 0.2) (layer "F.Cu") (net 3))
 (segment (start 83.058 159.2038) (end 83.2578 159.2038) (width 0.2) (layer "F.Cu") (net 3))
 (segment (start 91.1175 152.9172) (end 91.8468 152.9172) (width 0.2) (layer "F.Cu") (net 3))
 (segment (start 83.2578 159.2038) (end 83.312 159.258) (width 0.2) (layer "F.Cu") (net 3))
 (segment (start 81.375 162.4875) (end 83.7475 162.4875) (width 0.2) (layer "F.Cu") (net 3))
 (segment (start 87.75 153.1625) (end 88.25 153.1625) (width 0.2) (layer "F.Cu") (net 3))
 (segment (start 87.75 152.7) (end 87.75 153.1625) (width 0.2) (layer "F.Cu") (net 3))
 (segment (start 91.32 154.25) (end 92.02 154.25) (width 0.2) (layer "F.Cu") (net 3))
 (segment (start 87.1452 147.5972) (end 87.122 147.574) (width 0.2) (layer "F.Cu") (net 3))
 (segment (start 85.075 158.125) (end 86.751 158.125) (width 0.2) (layer "F.Cu") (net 3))
 (segment (start 87.2375 152.65) (end 87.7 152.65) (width 0.2) (layer "F.Cu") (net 3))
 (via (at 85.852 151.892) (size 0.6) (drill 0.3) (layers "F.Cu" "B.Cu") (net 3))
 (via (at 90.932 162.56) (size 0.6) (drill 0.3) (layers "F.Cu" "B.Cu") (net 3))
 (via (at 92.202 154.432) (size 0.6) (drill 0.3) (layers "F.Cu" "B.Cu") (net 3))
 (via (at 83.82 162.56) (size 0.6) (drill 0.3) (layers "F.Cu" "B.Cu") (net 3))
 (via (at 87.122 147.574) (size 0.6) (drill 0.3) (layers "F.Cu" "B.Cu") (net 3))
 (via (at 83.312 159.258) (size 0.6) (drill 0.3) (layers "F.Cu" "B.Cu") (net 3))
 (via (at 91.856 150.968) (size 0.6) (drill 0.3) (layers "F.Cu" "B.Cu") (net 3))
 (via (at 86.868 158.242) (size 0.6) (drill 0.3) (layers "F.Cu" "B.Cu") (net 3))
 (via (at 91.856 151.892) (size 0.6) (drill 0.3) (layers "F.Cu" "B.Cu") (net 3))
 (via (at 91.856 152.908) (size 0.6) (drill 0.3) (layers "F.Cu" "B.Cu") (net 3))
 (via (at 88.9 158.496) (size 0.6) (drill 0.3) (layers "F.Cu" "B.Cu") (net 3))
 (segment (start 80.75 152.93) (end 82.7214 150.9586) (width 0.2) (layer "F.Cu") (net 1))
 (segment (start 79.18 152.93) (end 80.75 152.93) (width 0.2) (layer "F.Cu") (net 1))
 (segment (start 82.7214 150.9586) (end 83.25 150.9586) (width 0.2) (layer "F.Cu") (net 1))
 (segment (start 78.25 152.25) (end 78.5 152.25) (width 0.2) (layer "F.Cu") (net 1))
 (segment (start 78.5 152.25) (end 79.18 152.93) (width 0.2) (layer "F.Cu") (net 1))
 (segment (start 85.75 152.93) (end 86.555 152.93) (width 0.2) (layer "F.Cu") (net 6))
 (segment (start 84.3139 152.93) (end 85.75 152.93) (width 0.2) (layer "F.Cu") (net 6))
 (segment (start 86.7875 153.1625) (end 87.25 153.1625) (width 0.2) (layer "F.Cu") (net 6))
 (segment (start 86.555 152.93) (end 86.7875 153.1625) (width 0.2) (layer "F.Cu") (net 6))
 (segment (start 84.2025 153.0414) (end 84.3139 152.93) (width 0.2) (layer "F.Cu") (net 6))
 (segment (start 86.872 152.15) (end 87.2375 152.15) (width 0.2) (layer "F.Cu") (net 2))
 (segment (start 86.0475 149.3922) (end 86.374 149.3922) (width 0.2) (layer "F.Cu") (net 2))
 (segment (start 78.25 149.5) (end 79.1528 148.5972) (width 0.2) (layer "F.Cu") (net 2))
 (segment (start 86.374 149.3922) (end 86.614 149.6322) (width 0.2) (layer "F.Cu") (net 2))
 (segment (start 79.1528 148.5972) (end 80.7975 148.5972) (width 0.2) (layer "F.Cu") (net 2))
 (segment (start 84.5 148.75) (end 85.1422 149.3922) (width 0.2) (layer "F.Cu") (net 2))
 (segment (start 82.7275 146.6672) (end 83.5475 146.6672) (width 0.2) (layer "F.Cu") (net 2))
 (segment (start 86.614 149.6322) (end 86.614 151.892) (width 0.2) (layer "F.Cu") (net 2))
 (segment (start 86.614 151.892) (end 86.872 152.15) (width 0.2) (layer "F.Cu") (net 2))
 (segment (start 80.7975 148.5972) (end 82.7275 146.6672) (width 0.2) (layer "F.Cu") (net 2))
 (segment (start 85.1422 149.3922) (end 86.0475 149.3922) (width 0.2) (layer "F.Cu") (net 2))
 (segment (start 89.2447 152.15) (end 90.4775 150.9172) (width 0.2) (layer "F.Cu") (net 4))
 (segment (start 88.0475 148.2372) (end 88.04335 148.24135) (width 0.2) (layer "F.Cu") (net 4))
 (segment (start 86.43 154.25) (end 85.75 153.57) (width 0.2) (layer "F.Cu") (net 4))
 (segment (start 92.456 153.416) (end 92.456 150.622) (width 0.2) (layer "F.Cu") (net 4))
 (segment (start 90.826701 150.368) (end 90.4775 150.717201) (width 0.2) (layer "F.Cu") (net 4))
 (segment (start 90.875 155.825) (end 90.68 155.63) (width 0.2) (layer "F.Cu") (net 4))
 (segment (start 92.456 150.622) (end 92.202 150.368) (width 0.2) (layer "F.Cu") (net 4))
 (segment (start 88.695901 148.2372) (end 88.0475 148.2372) (width 0.2) (layer "F.Cu") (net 4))
 (segment (start 87.25 151.6375) (end 87.25 149.1342) (width 0.2) (layer "F.Cu") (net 4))
 (segment (start 87.5325 148.7522) (end 88.0475 148.2372) (width 0.2) (layer "F.Cu") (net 4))
 (segment (start 90.68 154.25) (end 90.68 154.050001) (width 0.2) (layer "F.Cu") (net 4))
 (segment (start 92.202 150.368) (end 90.826701 150.368) (width 0.2) (layer "F.Cu") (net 4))
 (segment (start 88.04335 148.24135) (end 88.04335 149.5174) (width 0.2) (layer "F.Cu") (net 4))
 (segment (start 88.7625 152.65) (end 89.7447 152.65) (width 0.2) (layer "F.Cu") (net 4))
 (segment (start 92.202 153.67) (end 92.456 153.416) (width 0.2) (layer "F.Cu") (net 4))
 (segment (start 86.868 148.7522) (end 87.5325 148.7522) (width 0.2) (layer "F.Cu") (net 4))
 (segment (start 88.0215 149.53925) (end 88 149.53925) (width 0.2) (layer "F.Cu") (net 4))
 (segment (start 87.25 149.1342) (end 86.868 148.7522) (width 0.2) (layer "F.Cu") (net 4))
 (segment (start 88.7625 152.15) (end 89.2447 152.15) (width 0.2) (layer "F.Cu") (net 4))
 (segment (start 90.68 155.63) (end 90.68 154.25) (width 0.2) (layer "F.Cu") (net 4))
 (segment (start 90.826701 150.368) (end 88.695901 148.2372) (width 0.2) (layer "F.Cu") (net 4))
 (segment (start 91.060001 153.67) (end 92.202 153.67) (width 0.2) (layer "F.Cu") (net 4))
 (segment (start 86.0475 148.7522) (end 86.868 148.7522) (width 0.2) (layer "F.Cu") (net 4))
 (segment (start 90.4775 150.9172) (end 90.4775 151.9172) (width 0.2) (layer "F.Cu") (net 4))
 (segment (start 90.4775 150.717201) (end 90.4775 150.9172) (width 0.2) (layer "F.Cu") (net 4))
 (segment (start 88.04335 149.5174) (end 88.0215 149.53925) (width 0.2) (layer "F.Cu") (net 4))
 (segment (start 90.68 154.050001) (end 91.060001 153.67) (width 0.2) (layer "F.Cu") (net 4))
 (segment (start 90.4775 151.9172) (end 90.3988 151.9172) (width 0.2) (layer "F.Cu") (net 4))
 (segment (start 89.7447 152.65) (end 90.4775 151.9172) (width 0.2) (layer "F.Cu") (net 4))
 (segment (start 90.68 154.25) (end 86.43 154.25) (width 0.2) (layer "F.Cu") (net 4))
 (segment (start 90.61 160.69) (end 90.875 160.425) (width 0.2) (layer "F.Cu") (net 5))
 (segment (start 80.75 153.57) (end 81.7689 153.57) (width 0.2) (layer "F.Cu") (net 5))
 (segment (start 76.9068 155.790878) (end 77.447678 155.25) (width 0.2) (layer "F.Cu") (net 5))
 (segment (start 77.20642 160.425) (end 90.875 160.425) (width 0.2) (layer "F.Cu") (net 5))
 (segment (start 80.25 155.25) (end 80.75 154.75) (width 0.2) (layer "F.Cu") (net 5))
 (segment (start 80.75 154.75) (end 80.75 153.57) (width 0.2) (layer "F.Cu") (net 5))
 (segment (start 82.1078 149.2372) (end 80.7975 149.2372) (width 0.2) (layer "F.Cu") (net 5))
 (segment (start 76.9068 156.761) (end 76.9068 155.790878) (width 0.2) (layer "F.Cu") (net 5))
 (segment (start 81.7689 153.57) (end 82.2975 153.0414) (width 0.2) (layer "F.Cu") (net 5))
 (segment (start 77.8958 157.75) (end 76.9068 158.739) (width 0.2) (layer "F.Cu") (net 5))
 (segment (start 76.9068 160.12538) (end 77.20642 160.425) (width 0.2) (layer "F.Cu") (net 5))
 (segment (start 78.625 162.4875) (end 76.9068 160.7693) (width 0.2) (layer "F.Cu") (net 5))
 (segment (start 76.9068 160.7693) (end 76.9068 158.739) (width 0.2) (layer "F.Cu") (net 5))
 (segment (start 82.7769 153.0414) (end 83.8294 151.9889) (width 0.2) (layer "F.Cu") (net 5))
 (segment (start 83.8294 151.9889) (end 83.8294 149.9844) (width 0.2) (layer "F.Cu") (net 5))
 (segment (start 83.8294 149.9844) (end 82.595 148.75) (width 0.2) (layer "F.Cu") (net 5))
 (segment (start 77.447678 155.25) (end 80.25 155.25) (width 0.2) (layer "F.Cu") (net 5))
 (segment (start 82.2975 153.0414) (end 82.7769 153.0414) (width 0.2) (layer "F.Cu") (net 5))
 (segment (start 77.8958 157.75) (end 76.9068 156.761) (width 0.2) (layer "F.Cu") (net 5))
 (segment (start 90.61 161.75) (end 90.61 160.69) (width 0.2) (layer "F.Cu") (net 5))
 (segment (start 76.9068 158.739) (end 76.9068 160.12538) (width 0.2) (layer "F.Cu") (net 5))
 (segment (start 82.595 148.75) (end 82.1078 149.2372) (width 0.2) (layer "F.Cu") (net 5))
 (segment (start 87.75 151.6375) (end 87.75 150.2715) (width 0.2) (layer "F.Cu") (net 7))
 (segment (start 87.75 150.2715) (end 88 150.0215) (width 0.2) (layer "F.Cu") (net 7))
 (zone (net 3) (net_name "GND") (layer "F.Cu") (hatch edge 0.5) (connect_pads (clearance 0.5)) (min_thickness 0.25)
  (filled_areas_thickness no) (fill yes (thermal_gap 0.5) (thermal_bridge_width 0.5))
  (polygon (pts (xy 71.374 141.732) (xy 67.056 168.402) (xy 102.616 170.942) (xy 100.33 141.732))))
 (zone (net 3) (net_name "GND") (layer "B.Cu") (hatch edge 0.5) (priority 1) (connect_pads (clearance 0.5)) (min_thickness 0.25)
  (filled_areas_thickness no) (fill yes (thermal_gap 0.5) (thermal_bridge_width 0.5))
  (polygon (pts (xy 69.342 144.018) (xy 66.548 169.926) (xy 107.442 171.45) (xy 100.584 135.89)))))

